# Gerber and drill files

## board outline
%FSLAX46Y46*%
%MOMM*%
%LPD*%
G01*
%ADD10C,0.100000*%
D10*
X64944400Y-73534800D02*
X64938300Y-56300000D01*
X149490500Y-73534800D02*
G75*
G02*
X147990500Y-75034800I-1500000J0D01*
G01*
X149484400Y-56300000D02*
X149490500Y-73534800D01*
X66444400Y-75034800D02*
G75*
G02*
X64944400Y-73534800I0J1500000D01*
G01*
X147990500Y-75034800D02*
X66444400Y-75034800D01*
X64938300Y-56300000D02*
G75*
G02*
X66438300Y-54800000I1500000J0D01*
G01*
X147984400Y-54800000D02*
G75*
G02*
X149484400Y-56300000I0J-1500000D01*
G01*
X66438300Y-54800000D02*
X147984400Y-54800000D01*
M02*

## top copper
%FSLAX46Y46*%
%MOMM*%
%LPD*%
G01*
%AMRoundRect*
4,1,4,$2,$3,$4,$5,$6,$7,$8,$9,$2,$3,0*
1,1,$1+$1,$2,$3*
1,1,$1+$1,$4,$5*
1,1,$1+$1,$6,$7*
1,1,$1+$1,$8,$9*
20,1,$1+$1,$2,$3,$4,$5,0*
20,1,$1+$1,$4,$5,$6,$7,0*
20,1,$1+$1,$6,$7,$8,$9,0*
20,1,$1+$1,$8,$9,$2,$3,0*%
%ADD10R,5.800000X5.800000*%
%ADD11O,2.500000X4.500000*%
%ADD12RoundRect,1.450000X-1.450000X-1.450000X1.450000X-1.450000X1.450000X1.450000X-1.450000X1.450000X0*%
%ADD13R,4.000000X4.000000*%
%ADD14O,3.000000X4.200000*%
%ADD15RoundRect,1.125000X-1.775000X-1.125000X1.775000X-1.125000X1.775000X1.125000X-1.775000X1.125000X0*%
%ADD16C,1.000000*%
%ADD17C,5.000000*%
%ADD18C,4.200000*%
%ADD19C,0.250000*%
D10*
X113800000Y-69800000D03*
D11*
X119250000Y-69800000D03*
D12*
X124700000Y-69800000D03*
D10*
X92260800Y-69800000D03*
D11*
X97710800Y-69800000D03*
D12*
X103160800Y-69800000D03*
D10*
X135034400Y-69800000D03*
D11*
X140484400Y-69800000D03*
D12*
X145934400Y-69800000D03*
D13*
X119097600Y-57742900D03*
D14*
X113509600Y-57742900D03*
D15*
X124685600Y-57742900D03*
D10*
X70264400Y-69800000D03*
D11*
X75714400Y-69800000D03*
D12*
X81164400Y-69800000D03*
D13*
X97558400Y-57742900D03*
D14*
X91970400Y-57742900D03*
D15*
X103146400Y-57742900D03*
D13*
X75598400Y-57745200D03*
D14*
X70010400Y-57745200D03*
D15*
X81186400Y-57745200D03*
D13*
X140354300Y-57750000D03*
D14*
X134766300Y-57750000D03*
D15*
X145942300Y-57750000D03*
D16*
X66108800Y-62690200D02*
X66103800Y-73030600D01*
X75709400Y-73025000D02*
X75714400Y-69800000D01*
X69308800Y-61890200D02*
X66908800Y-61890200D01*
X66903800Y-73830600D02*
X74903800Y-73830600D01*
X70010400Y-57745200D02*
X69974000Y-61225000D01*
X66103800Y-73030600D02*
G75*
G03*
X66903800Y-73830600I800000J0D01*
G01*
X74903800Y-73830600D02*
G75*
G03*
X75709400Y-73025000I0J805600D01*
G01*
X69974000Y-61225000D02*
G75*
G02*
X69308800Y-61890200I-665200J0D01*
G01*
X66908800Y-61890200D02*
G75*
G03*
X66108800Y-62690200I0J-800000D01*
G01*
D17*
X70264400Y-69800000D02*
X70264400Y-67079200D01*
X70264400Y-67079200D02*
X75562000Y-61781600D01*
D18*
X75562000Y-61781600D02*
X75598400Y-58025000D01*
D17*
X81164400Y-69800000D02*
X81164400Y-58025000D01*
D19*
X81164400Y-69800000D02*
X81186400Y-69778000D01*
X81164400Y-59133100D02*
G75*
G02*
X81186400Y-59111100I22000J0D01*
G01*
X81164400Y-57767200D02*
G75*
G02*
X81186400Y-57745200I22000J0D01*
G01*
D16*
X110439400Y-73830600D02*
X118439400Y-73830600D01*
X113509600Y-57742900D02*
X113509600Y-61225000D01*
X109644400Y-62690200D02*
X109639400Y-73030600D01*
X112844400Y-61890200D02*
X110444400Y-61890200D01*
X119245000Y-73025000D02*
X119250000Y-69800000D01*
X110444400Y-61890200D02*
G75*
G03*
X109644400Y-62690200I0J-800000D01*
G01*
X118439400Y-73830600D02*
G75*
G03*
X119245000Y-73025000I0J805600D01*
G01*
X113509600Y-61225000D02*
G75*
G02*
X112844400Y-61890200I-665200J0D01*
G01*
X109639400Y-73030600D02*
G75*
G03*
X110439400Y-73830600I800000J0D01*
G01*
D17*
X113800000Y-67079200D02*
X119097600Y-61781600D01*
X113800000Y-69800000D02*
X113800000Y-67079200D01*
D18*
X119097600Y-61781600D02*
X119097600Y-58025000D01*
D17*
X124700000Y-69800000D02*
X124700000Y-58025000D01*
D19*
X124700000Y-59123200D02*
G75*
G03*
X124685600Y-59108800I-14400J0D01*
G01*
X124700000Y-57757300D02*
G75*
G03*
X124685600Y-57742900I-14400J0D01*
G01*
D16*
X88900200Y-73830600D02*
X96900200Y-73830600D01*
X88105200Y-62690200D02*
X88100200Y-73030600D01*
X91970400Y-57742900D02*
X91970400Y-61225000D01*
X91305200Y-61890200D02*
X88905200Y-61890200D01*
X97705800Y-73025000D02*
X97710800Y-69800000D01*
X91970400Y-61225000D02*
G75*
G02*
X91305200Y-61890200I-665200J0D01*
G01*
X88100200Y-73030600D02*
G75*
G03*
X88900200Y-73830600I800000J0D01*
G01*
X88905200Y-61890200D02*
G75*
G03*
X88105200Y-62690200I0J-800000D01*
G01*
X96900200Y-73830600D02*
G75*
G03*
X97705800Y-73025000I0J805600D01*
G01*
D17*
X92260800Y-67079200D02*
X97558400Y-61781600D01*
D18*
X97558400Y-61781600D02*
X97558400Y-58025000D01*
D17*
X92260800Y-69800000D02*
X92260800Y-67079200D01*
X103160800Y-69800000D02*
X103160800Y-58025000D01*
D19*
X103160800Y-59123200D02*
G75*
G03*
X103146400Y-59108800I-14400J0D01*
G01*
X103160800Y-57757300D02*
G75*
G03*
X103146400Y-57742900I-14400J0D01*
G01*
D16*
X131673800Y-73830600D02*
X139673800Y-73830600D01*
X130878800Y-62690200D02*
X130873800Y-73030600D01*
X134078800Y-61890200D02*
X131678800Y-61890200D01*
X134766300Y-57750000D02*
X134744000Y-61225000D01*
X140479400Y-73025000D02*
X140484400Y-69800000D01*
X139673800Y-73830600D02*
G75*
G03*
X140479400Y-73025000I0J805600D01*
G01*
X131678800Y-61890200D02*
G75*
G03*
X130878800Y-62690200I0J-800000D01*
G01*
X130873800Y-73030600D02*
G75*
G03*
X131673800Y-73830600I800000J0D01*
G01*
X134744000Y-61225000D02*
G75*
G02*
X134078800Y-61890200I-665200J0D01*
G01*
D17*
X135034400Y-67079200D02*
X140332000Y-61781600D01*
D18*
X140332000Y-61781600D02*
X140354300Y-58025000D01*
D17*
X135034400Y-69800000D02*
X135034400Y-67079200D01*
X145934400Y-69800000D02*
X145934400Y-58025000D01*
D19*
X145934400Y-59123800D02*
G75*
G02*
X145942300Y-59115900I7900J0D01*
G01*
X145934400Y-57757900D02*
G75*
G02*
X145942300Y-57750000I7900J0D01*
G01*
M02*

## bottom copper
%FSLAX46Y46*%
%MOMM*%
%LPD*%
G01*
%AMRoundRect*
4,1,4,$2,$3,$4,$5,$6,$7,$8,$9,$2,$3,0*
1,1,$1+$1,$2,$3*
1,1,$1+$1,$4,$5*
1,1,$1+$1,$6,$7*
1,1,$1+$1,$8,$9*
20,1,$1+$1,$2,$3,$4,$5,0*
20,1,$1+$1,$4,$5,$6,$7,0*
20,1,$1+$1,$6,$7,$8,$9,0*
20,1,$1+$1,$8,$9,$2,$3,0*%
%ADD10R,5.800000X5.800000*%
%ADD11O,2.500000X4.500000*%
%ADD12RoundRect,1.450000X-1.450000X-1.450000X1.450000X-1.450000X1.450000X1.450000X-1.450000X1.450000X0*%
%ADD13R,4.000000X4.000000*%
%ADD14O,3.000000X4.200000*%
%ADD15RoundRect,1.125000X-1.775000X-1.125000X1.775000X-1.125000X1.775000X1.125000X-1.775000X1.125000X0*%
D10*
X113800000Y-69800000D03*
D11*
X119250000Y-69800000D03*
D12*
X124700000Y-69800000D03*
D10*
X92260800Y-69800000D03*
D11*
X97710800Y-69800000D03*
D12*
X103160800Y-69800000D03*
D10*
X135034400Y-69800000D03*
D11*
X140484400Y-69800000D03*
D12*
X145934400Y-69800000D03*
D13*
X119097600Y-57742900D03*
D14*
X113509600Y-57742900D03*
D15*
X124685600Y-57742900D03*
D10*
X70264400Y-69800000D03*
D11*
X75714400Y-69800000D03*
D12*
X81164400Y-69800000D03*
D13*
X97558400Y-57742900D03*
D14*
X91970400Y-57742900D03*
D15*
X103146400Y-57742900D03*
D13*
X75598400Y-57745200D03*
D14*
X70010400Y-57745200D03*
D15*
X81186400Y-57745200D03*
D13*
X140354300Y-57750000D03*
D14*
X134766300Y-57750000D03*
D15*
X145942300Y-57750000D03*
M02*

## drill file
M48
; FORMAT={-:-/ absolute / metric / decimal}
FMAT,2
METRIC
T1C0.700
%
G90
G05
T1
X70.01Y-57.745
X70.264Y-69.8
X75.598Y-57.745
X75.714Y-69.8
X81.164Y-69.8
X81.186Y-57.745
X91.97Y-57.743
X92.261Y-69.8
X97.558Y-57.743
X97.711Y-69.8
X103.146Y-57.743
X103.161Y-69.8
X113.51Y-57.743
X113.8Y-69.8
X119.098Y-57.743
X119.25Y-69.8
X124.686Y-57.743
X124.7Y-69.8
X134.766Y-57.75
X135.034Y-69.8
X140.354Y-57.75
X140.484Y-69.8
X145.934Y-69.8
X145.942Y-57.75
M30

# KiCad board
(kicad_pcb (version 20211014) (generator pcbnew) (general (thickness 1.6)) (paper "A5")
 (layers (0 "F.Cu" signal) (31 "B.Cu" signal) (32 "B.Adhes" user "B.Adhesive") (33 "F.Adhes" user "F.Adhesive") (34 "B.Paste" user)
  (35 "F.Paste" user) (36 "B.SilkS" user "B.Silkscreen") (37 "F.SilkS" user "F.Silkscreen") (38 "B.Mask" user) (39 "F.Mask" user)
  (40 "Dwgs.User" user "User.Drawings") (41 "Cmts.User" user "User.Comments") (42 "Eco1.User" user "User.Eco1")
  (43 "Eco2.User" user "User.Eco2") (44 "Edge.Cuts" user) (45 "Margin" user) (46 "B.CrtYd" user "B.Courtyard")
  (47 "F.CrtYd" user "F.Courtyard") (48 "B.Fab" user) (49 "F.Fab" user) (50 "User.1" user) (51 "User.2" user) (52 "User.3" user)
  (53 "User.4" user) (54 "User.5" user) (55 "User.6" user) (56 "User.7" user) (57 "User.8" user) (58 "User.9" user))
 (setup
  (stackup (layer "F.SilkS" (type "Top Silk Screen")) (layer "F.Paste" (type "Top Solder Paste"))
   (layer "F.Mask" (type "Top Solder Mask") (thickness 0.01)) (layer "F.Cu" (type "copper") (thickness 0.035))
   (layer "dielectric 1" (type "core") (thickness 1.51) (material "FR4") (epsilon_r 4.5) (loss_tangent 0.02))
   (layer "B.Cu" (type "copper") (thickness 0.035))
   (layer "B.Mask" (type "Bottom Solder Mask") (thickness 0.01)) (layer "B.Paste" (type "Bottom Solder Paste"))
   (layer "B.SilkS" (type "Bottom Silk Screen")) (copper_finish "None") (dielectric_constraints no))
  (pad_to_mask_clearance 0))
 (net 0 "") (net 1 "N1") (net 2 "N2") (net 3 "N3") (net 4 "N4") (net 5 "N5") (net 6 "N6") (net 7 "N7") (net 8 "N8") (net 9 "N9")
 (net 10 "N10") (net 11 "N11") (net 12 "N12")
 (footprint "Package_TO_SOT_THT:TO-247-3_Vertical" (layer "F.Cu") (at 113.8 69.8)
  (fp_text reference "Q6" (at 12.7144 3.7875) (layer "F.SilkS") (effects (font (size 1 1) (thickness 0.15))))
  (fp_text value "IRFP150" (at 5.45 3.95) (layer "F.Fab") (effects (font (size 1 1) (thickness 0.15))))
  (pad "1" thru_hole rect (at 0 0) (size 5.8 5.8) (drill 0.7) (layers *.Cu *.Mask) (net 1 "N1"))
  (pad "2" thru_hole oval (at 5.45 0) (size 2.5 4.5) (drill 0.7) (layers *.Cu *.Mask) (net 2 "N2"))
  (pad "3" thru_hole roundrect (at 10.9 0) (size 5.8 5.8) (drill 0.7) (layers *.Cu *.Mask) (roundrect_rratio 0.25) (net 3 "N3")))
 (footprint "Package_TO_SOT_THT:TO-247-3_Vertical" (layer "F.Cu") (at 92.2608 69.8)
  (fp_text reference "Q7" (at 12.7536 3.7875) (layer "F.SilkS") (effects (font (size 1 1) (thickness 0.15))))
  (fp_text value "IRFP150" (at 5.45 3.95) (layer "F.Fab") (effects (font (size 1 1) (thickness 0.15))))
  (pad "1" thru_hole rect (at 0 0) (size 5.8 5.8) (drill 0.7) (layers *.Cu *.Mask) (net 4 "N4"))
  (pad "2" thru_hole oval (at 5.45 0) (size 2.5 4.5) (drill 0.7) (layers *.Cu *.Mask) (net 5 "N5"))
  (pad "3" thru_hole roundrect (at 10.9 0) (size 5.8 5.8) (drill 0.7) (layers *.Cu *.Mask) (roundrect_rratio 0.25) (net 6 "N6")))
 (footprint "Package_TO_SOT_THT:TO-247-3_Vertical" (layer "F.Cu") (at 135.0344 69.8)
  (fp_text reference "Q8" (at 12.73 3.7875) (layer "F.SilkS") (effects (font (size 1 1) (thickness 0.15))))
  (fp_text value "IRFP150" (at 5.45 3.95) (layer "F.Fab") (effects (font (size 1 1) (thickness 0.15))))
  (pad "1" thru_hole rect (at 0 0) (size 5.8 5.8) (drill 0.7) (layers *.Cu *.Mask) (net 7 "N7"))
  (pad "2" thru_hole oval (at 5.45 0) (size 2.5 4.5) (drill 0.7) (layers *.Cu *.Mask) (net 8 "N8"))
  (pad "3" thru_hole roundrect (at 10.9 0) (size 5.8 5.8) (drill 0.7) (layers *.Cu *.Mask) (roundrect_rratio 0.25) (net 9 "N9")))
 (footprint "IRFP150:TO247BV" (layer "F.Cu") (at 119.0976 54.8219)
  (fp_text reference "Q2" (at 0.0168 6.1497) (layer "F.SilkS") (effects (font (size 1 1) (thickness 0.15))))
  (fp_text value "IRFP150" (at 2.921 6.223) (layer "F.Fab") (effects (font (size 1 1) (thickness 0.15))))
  (pad "D" thru_hole rect locked (at 0 2.921) (size 4 4) (drill 0.7) (layers *.Cu *.Mask) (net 1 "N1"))
  (pad "G" thru_hole oval locked (at -5.588 2.921) (size 3 4.2) (drill 0.7) (layers *.Cu *.Mask) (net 2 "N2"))
  (pad "S" thru_hole roundrect locked (at 5.588 2.921) (size 5.8 4.5) (drill 0.7) (layers *.Cu *.Mask) (roundrect_rratio 0.25) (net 3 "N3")))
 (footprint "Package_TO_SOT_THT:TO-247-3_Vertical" (layer "F.Cu") (at 70.2644 69.8)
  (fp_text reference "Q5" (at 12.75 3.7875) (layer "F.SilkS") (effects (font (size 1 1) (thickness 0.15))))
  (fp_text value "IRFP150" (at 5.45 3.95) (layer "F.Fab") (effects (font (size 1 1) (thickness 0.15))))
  (pad "1" thru_hole rect (at 0 0) (size 5.8 5.8) (drill 0.7) (layers *.Cu *.Mask) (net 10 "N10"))
  (pad "2" thru_hole oval (at 5.45 0) (size 2.5 4.5) (drill 0.7) (layers *.Cu *.Mask) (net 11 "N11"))
  (pad "3" thru_hole roundrect (at 10.9 0) (size 5.8 5.8) (drill 0.7) (layers *.Cu *.Mask) (roundrect_rratio 0.25) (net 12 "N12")))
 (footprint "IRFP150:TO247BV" (layer "F.Cu") (at 97.5584 54.8219)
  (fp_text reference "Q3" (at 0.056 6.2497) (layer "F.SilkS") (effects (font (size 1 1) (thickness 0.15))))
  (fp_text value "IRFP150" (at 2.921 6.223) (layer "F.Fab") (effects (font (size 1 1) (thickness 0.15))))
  (pad "D" thru_hole rect locked (at 0 2.921) (size 4 4) (drill 0.7) (layers *.Cu *.Mask) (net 4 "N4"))
  (pad "G" thru_hole oval locked (at -5.588 2.921) (size 3 4.2) (drill 0.7) (layers *.Cu *.Mask) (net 5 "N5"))
  (pad "S" thru_hole roundrect locked (at 5.588 2.921) (size 5.8 4.5) (drill 0.7) (layers *.Cu *.Mask) (roundrect_rratio 0.25) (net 6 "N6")))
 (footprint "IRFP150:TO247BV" (layer "F.Cu") (at 75.5984 54.8242)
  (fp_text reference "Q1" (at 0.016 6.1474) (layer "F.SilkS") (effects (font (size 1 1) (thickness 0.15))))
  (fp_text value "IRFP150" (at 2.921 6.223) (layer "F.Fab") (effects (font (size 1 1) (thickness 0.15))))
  (pad "D" thru_hole rect locked (at 0 2.921) (size 4 4) (drill 0.7) (layers *.Cu *.Mask) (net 10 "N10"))
  (pad "G" thru_hole oval locked (at -5.588 2.921) (size 3 4.2) (drill 0.7) (layers *.Cu *.Mask) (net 11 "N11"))
  (pad "S" thru_hole roundrect locked (at 5.588 2.921) (size 5.8 4.5) (drill 0.7) (layers *.Cu *.Mask) (roundrect_rratio 0.25)
   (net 12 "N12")))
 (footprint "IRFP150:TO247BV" (layer "F.Cu") (at 140.3543 54.829)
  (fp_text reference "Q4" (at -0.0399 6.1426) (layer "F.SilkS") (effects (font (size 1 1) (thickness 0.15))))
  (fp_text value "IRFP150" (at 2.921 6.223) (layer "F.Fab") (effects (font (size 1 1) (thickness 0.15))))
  (pad "D" thru_hole rect locked (at 0 2.921) (size 4 4) (drill 0.7) (layers *.Cu *.Mask) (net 7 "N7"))
  (pad "G" thru_hole oval locked (at -5.588 2.921) (size 3 4.2) (drill 0.7) (layers *.Cu *.Mask) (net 8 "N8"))
  (pad "S" thru_hole roundrect locked (at 5.588 2.921) (size 5.8 4.5) (drill 0.7) (layers *.Cu *.Mask) (roundrect_rratio 0.25) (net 9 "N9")))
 (gr_line (start 64.9444 73.5348) (end 64.9383 56.3) (layer "Edge.Cuts") (width 0.1))
 (gr_arc (start 149.4905 73.5348) (mid 149.05116 74.59546) (end 147.9905 75.0348) (layer "Edge.Cuts") (width 0.1))
 (gr_line (start 149.4844 56.3) (end 149.4905 73.5348) (layer "Edge.Cuts") (width 0.1))
 (gr_arc (start 66.4444 75.0348) (mid 65.38374 74.59546) (end 64.9444 73.5348) (layer "Edge.Cuts") (width 0.1))
 (gr_line (start 147.9905 75.0348) (end 66.4444 75.0348) (layer "Edge.Cuts") (width 0.1))
 (gr_arc (start 64.9383 56.3) (mid 65.37764 55.23934) (end 66.4383 54.8) (layer "Edge.Cuts") (width 0.1))
 (gr_arc (start 147.9844 54.8) (mid 149.04506 55.23934) (end 149.4844 56.3) (layer "Edge.Cuts") (width 0.1))
 (gr_line (start 66.4383 54.8) (end 147.9844 54.8) (layer "Edge.Cuts") (width 0.1))
 (segment (start 66.1088 62.6902) (end 66.1038 73.0306) (width 1) (layer "F.Cu") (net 11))
 (segment (start 75.7094 73.025) (end 75.7144 69.8) (width 1) (layer "F.Cu") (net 11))
 (segment (start 69.3088 61.8902) (end 66.9088 61.8902) (width 1) (layer "F.Cu") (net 11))
 (segment (start 66.9038 73.8306) (end 74.9038 73.8306) (width 1) (layer "F.Cu") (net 11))
 (segment (start 70.0104 57.7452) (end 69.974 61.225) (width 1) (layer "F.Cu") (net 11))
 (arc (start 66.1038 73.0306) (mid 66.338115 73.596285) (end 66.9038 73.8306) (width 1) (layer "F.Cu") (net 11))
 (arc (start 74.9038 73.8306) (mid 75.473445 73.594645) (end 75.7094 73.025) (width 1) (layer "F.Cu") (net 11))
 (arc (start 69.974 61.225) (mid 69.779167 61.695367) (end 69.3088 61.8902) (width 1) (layer "F.Cu") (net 11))
 (arc (start 66.9088 61.8902) (mid 66.343115 62.124515) (end 66.1088 62.6902) (width 1) (layer "F.Cu") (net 11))
 (segment (start 70.2644 69.8) (end 70.2644 67.0792) (width 5) (layer "F.Cu") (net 10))
 (segment (start 70.2644 67.0792) (end 75.562 61.7816) (width 5) (layer "F.Cu") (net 10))
 (segment (start 75.562 61.7816) (end 75.5984 58.025) (width 4.2) (layer "F.Cu") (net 10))
 (segment (start 81.1644 69.8) (end 81.1644 58.025) (width 5) (layer "F.Cu") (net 12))
 (segment (start 81.1644 69.8) (end 81.1864 69.778) (width 0.25) (layer "F.Cu") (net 12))
 (arc (start 81.1644 59.1331) (mid 81.170844 59.117544) (end 81.1864 59.1111) (width 0.25) (layer "F.Cu") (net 12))
 (arc (start 81.1644 57.7672) (mid 81.170844 57.751644) (end 81.1864 57.7452) (width 0.25) (layer "F.Cu") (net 12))
 (segment (start 110.4394 73.8306) (end 118.4394 73.8306) (width 1) (layer "F.Cu") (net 2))
 (segment (start 113.5096 57.7429) (end 113.5096 61.225) (width 1) (layer "F.Cu") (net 2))
 (segment (start 109.6444 62.6902) (end 109.6394 73.0306) (width 1) (layer "F.Cu") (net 2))
 (segment (start 112.8444 61.8902) (end 110.4444 61.8902) (width 1) (layer "F.Cu") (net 2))
 (segment (start 119.245 73.025) (end 119.25 69.8) (width 1) (layer "F.Cu") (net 2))
 (arc (start 110.4444 61.8902) (mid 109.878715 62.124515) (end 109.6444 62.6902) (width 1) (layer "F.Cu") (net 2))
 (arc (start 118.4394 73.8306) (mid 119.009045 73.594645) (end 119.245 73.025) (width 1) (layer "F.Cu") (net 2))
 (arc (start 113.5096 61.225) (mid 113.314767 61.695367) (end 112.8444 61.8902) (width 1) (layer "F.Cu") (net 2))
 (arc (start 109.6394 73.0306) (mid 109.873715 73.596285) (end 110.4394 73.8306) (width 1) (layer "F.Cu") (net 2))
 (segment (start 113.8 67.0792) (end 119.0976 61.7816) (width 5) (layer "F.Cu") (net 1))
 (segment (start 113.8 69.8) (end 113.8 67.0792) (width 5) (layer "F.Cu") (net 1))
 (segment (start 119.0976 61.7816) (end 119.0976 58.025) (width 4.2) (layer "F.Cu") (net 1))
 (segment (start 124.7 69.8) (end 124.7 58.025) (width 5) (layer "F.Cu") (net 3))
 (arc (start 124.7 59.1232) (mid 124.695782 59.113018) (end 124.6856 59.1088) (width 0.25) (layer "F.Cu") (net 3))
 (arc (start 124.7 57.7573) (mid 124.695782 57.747118) (end 124.6856 57.7429) (width 0.25) (layer "F.Cu") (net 3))
 (segment (start 88.9002 73.8306) (end 96.9002 73.8306) (width 1) (layer "F.Cu") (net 5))
 (segment (start 88.1052 62.6902) (end 88.1002 73.0306) (width 1) (layer "F.Cu") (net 5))
 (segment (start 91.9704 57.7429) (end 91.9704 61.225) (width 1) (layer "F.Cu") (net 5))
 (segment (start 91.3052 61.8902) (end 88.9052 61.8902) (width 1) (layer "F.Cu") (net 5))
 (segment (start 97.7058 73.025) (end 97.7108 69.8) (width 1) (layer "F.Cu") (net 5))
 (arc (start 91.9704 61.225) (mid 91.775567 61.695367) (end 91.3052 61.8902) (width 1) (layer "F.Cu") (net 5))
 (arc (start 88.1002 73.0306) (mid 88.334515 73.596285) (end 88.9002 73.8306) (width 1) (layer "F.Cu") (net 5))
 (arc (start 88.9052 61.8902) (mid 88.339515 62.124515) (end 88.1052 62.6902) (width 1) (layer "F.Cu") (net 5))
 (arc (start 96.9002 73.8306) (mid 97.469845 73.594645) (end 97.7058 73.025) (width 1) (layer "F.Cu") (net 5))
 (segment (start 92.2608 67.0792) (end 97.5584 61.7816) (width 5) (layer "F.Cu") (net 4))
 (segment (start 97.5584 61.7816) (end 97.5584 58.025) (width 4.2) (layer "F.Cu") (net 4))
 (segment (start 92.2608 69.8) (end 92.2608 67.0792) (width 5) (layer "F.Cu") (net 4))
 (segment (start 103.1608 69.8) (end 103.1608 58.025) (width 5) (layer "F.Cu") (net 6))
 (arc (start 103.1608 59.1232) (mid 103.156582 59.113018) (end 103.1464 59.1088) (width 0.25) (layer "F.Cu") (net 6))
 (arc (start 103.1608 57.7573) (mid 103.156582 57.747118) (end 103.1464 57.7429) (width 0.25) (layer "F.Cu") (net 6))
 (segment (start 131.6738 73.8306) (end 139.6738 73.8306) (width 1) (layer "F.Cu") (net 8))
 (segment (start 130.8788 62.6902) (end 130.8738 73.0306) (width 1) (layer "F.Cu") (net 8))
 (segment (start 134.0788 61.8902) (end 131.6788 61.8902) (width 1) (layer "F.Cu") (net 8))
 (segment (start 134.7663 57.75) (end 134.744 61.225) (width 1) (layer "F.Cu") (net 8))
 (segment (start 140.4794 73.025) (end 140.4844 69.8) (width 1) (layer "F.Cu") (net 8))
 (arc (start 139.6738 73.8306) (mid 140.243445 73.594645) (end 140.4794 73.025) (width 1) (layer "F.Cu") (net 8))
 (arc (start 131.6788 61.8902) (mid 131.113115 62.124515) (end 130.8788 62.6902) (width 1) (layer "F.Cu") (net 8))
 (arc (start 130.8738 73.0306) (mid 131.108115 73.596285) (end 131.6738 73.8306) (width 1) (layer "F.Cu") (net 8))
 (arc (start 134.744 61.225) (mid 134.549167 61.695367) (end 134.0788 61.8902) (width 1) (layer "F.Cu") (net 8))
 (segment (start 135.0344 67.0792) (end 140.332 61.7816) (width 5) (layer "F.Cu") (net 7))
 (segment (start 140.332 61.7816) (end 140.3543 58.025) (width 4.2) (layer "F.Cu") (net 7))
 (segment (start 135.0344 69.8) (end 135.0344 67.0792) (width 5) (layer "F.Cu") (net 7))
 (segment (start 145.9344 69.8) (end 145.9344 58.025) (width 5) (layer "F.Cu") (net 9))
 (arc (start 145.9344 59.1238) (mid 145.936714 59.118214) (end 145.9423 59.1159) (width 0.25) (layer "F.Cu") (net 9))
 (arc (start 145.9344 57.7579) (mid 145.936714 57.752314) (end 145.9423 57.75) (width 0.25) (layer "F.Cu") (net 9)))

